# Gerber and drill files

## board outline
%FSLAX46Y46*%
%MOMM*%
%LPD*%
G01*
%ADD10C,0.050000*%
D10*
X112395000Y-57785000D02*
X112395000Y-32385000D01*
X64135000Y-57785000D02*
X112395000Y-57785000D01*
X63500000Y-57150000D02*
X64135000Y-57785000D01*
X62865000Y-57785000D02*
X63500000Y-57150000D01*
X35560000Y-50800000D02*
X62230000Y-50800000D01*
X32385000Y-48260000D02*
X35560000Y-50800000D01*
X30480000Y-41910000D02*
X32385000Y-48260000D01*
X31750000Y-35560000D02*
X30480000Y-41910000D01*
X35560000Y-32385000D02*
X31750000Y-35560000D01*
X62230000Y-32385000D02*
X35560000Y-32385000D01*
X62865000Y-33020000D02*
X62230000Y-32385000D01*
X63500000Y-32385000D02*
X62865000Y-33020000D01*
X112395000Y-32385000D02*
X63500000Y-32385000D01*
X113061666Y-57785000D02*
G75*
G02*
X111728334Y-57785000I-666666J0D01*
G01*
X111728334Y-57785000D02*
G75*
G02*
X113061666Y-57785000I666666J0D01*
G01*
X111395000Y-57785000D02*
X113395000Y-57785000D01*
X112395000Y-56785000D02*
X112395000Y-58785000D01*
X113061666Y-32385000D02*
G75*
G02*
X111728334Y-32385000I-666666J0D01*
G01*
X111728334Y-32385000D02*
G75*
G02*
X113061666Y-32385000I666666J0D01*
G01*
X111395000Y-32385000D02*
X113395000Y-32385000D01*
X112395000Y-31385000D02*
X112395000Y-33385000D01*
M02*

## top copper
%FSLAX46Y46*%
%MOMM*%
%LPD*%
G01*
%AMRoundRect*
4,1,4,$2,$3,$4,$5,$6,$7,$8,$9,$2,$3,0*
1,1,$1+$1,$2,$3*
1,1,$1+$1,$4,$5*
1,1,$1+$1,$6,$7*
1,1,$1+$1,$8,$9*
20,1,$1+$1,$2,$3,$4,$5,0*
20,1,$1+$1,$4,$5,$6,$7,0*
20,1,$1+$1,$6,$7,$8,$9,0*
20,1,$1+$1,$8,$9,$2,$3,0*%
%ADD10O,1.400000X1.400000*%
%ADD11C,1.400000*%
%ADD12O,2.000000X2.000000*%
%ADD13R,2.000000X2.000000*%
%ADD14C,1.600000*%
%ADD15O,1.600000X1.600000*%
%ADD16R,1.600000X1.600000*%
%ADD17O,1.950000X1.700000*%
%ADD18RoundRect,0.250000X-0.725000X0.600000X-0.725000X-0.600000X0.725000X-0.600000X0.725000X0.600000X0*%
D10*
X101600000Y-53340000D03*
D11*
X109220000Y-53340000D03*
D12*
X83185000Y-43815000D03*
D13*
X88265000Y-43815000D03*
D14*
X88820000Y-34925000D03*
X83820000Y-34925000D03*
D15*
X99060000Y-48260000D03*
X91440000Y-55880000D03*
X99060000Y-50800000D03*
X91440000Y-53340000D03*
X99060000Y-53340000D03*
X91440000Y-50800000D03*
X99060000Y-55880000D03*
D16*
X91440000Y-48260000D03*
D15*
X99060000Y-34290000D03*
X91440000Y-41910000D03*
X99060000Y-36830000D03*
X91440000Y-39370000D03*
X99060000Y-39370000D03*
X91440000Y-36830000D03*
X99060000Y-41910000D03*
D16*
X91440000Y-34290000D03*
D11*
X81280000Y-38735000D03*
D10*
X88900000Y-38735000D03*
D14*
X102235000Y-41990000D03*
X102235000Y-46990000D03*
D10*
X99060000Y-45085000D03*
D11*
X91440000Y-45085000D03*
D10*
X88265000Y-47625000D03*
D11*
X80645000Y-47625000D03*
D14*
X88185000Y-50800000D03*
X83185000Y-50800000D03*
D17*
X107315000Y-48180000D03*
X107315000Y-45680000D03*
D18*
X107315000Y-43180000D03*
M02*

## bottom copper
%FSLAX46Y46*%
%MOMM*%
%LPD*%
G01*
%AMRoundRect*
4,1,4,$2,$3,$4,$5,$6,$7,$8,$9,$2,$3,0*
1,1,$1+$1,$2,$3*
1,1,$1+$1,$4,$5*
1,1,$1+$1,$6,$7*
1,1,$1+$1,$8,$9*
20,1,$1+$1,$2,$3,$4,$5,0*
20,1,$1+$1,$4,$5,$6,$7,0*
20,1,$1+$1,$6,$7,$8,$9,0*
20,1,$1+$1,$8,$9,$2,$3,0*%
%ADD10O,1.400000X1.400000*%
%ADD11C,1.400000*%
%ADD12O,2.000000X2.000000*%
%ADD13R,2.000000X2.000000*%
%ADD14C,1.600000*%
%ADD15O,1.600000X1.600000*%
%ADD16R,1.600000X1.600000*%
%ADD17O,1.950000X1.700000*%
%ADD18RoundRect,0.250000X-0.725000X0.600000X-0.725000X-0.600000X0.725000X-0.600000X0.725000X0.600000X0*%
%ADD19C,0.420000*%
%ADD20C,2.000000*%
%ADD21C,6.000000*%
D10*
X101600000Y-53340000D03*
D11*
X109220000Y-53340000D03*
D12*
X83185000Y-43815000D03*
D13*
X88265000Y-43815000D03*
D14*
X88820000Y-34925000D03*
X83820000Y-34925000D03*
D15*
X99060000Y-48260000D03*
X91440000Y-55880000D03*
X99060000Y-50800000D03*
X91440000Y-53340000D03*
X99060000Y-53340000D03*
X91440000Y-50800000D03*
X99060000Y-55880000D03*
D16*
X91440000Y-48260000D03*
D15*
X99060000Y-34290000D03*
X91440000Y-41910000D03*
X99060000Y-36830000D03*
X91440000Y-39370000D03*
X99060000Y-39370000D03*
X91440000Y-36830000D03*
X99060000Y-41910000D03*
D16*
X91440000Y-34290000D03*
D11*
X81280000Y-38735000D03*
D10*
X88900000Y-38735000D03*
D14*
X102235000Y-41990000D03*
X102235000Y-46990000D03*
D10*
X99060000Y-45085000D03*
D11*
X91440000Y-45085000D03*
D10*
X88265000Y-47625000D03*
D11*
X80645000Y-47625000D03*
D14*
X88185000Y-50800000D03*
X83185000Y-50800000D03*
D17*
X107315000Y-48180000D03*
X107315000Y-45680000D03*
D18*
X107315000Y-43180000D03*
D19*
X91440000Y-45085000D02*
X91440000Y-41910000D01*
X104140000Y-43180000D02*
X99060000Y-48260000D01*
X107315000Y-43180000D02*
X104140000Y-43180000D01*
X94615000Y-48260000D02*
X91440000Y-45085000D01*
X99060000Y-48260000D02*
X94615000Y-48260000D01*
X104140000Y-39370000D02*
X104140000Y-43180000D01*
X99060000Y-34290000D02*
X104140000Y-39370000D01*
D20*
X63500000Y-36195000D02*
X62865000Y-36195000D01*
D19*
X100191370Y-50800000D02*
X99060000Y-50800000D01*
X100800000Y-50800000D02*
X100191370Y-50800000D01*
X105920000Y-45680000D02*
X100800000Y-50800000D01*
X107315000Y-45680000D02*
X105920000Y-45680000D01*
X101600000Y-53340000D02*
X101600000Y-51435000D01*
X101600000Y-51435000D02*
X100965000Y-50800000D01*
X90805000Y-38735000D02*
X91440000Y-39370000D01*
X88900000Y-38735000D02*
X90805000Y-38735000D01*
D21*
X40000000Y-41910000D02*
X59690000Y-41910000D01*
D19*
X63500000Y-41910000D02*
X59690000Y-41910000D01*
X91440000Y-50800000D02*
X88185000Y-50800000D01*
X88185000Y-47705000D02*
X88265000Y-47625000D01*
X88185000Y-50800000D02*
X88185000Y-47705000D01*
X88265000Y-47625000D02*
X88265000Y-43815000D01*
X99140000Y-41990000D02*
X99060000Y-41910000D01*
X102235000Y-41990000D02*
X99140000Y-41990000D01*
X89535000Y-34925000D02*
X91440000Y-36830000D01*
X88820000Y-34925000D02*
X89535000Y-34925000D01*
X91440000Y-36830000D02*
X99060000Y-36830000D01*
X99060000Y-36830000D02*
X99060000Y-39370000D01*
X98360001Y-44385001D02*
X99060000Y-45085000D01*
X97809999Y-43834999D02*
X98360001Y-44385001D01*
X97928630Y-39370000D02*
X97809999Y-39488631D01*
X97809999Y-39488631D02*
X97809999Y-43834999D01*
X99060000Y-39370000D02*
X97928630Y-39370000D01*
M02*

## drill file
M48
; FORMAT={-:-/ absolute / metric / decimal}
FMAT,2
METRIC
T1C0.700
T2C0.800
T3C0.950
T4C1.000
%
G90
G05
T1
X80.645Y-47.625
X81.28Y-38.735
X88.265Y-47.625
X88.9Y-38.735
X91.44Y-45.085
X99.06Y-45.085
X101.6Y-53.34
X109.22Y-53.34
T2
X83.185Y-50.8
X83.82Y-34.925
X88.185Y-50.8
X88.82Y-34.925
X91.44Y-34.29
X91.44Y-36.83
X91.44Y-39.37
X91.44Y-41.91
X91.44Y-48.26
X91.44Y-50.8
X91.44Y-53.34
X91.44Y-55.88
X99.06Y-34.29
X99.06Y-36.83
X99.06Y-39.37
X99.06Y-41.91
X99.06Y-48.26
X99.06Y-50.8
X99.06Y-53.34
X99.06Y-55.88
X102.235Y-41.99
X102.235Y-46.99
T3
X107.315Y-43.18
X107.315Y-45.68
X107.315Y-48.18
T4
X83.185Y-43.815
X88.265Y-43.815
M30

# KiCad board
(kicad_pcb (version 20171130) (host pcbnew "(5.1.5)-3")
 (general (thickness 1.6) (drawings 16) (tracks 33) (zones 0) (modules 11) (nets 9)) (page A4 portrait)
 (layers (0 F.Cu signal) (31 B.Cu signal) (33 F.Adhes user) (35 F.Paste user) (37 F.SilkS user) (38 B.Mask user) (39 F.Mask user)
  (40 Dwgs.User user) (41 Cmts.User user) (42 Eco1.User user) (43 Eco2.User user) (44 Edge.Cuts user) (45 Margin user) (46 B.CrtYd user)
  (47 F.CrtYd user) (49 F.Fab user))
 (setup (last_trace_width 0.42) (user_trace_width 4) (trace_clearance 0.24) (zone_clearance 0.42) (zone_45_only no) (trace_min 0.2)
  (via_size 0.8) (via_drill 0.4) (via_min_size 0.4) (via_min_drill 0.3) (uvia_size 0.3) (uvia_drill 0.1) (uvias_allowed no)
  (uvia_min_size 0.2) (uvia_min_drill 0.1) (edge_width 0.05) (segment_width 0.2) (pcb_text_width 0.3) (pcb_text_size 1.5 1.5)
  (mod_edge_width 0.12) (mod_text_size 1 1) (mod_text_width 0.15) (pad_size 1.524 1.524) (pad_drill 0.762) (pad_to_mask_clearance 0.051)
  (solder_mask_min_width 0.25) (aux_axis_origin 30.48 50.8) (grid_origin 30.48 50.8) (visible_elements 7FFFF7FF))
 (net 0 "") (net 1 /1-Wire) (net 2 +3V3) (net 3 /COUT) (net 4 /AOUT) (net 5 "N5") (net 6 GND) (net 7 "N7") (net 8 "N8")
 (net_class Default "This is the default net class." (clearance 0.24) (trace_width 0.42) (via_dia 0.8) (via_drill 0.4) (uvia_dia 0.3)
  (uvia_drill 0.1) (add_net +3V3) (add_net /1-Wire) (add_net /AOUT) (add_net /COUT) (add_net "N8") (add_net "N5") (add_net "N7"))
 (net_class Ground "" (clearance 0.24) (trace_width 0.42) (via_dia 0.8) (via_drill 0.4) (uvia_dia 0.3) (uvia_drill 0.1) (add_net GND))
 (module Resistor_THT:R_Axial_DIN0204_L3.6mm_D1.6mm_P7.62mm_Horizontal (layer F.Cu) (at 109.22 53.34 180)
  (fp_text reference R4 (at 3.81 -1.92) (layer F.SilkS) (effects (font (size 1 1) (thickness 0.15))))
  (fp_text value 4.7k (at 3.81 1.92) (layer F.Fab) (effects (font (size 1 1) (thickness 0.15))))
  (pad 2 thru_hole oval (at 7.62 0 180) (size 1.4 1.4) (drill 0.7) (layers *.Cu *.Mask) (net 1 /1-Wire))
  (pad 1 thru_hole circle (at 0 0 180) (size 1.4 1.4) (drill 0.7) (layers *.Cu *.Mask) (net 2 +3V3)))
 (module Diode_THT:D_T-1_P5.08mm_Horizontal (layer F.Cu) (at 88.265 43.815 180)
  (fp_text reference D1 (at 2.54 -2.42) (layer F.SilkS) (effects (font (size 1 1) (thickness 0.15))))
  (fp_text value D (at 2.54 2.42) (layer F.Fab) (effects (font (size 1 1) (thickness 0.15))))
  (pad 2 thru_hole oval (at 5.08 0 180) (size 2 2) (drill 1) (layers *.Cu *.Mask) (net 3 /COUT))
  (pad 1 thru_hole rect (at 0 0 180) (size 2 2) (drill 1) (layers *.Cu *.Mask) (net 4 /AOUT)))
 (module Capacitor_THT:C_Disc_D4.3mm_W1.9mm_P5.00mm (layer F.Cu) (at 83.82 34.925)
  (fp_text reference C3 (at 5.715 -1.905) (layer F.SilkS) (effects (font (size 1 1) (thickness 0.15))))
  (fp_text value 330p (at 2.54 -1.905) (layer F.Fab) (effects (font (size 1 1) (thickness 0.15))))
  (pad 2 thru_hole circle (at 5 0) (size 1.6 1.6) (drill 0.8) (layers *.Cu *.Mask) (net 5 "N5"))
  (pad 1 thru_hole circle (at 0 0) (size 1.6 1.6) (drill 0.8) (layers *.Cu *.Mask) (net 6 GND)))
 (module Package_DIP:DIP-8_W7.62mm (layer F.Cu) (at 91.44 48.26)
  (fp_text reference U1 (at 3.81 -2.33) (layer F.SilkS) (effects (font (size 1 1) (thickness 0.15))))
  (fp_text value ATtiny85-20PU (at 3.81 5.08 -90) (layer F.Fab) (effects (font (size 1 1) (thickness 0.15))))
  (pad 8 thru_hole oval (at 7.62 0) (size 1.6 1.6) (drill 0.8) (layers *.Cu *.Mask) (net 2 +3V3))
  (pad 4 thru_hole oval (at 0 7.62) (size 1.6 1.6) (drill 0.8) (layers *.Cu *.Mask) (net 6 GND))
  (pad 7 thru_hole oval (at 7.62 2.54) (size 1.6 1.6) (drill 0.8) (layers *.Cu *.Mask) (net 1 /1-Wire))
  (pad 3 thru_hole oval (at 0 5.08) (size 1.6 1.6) (drill 0.8) (layers *.Cu *.Mask) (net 6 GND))
  (pad 6 thru_hole oval (at 7.62 5.08) (size 1.6 1.6) (drill 0.8) (layers *.Cu *.Mask))
  (pad 2 thru_hole oval (at 0 2.54) (size 1.6 1.6) (drill 0.8) (layers *.Cu *.Mask) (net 4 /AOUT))
  (pad 5 thru_hole oval (at 7.62 7.62) (size 1.6 1.6) (drill 0.8) (layers *.Cu *.Mask))
  (pad 1 thru_hole rect (at 0 0) (size 1.6 1.6) (drill 0.8) (layers *.Cu *.Mask)))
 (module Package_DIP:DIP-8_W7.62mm (layer F.Cu) (at 91.44 34.29)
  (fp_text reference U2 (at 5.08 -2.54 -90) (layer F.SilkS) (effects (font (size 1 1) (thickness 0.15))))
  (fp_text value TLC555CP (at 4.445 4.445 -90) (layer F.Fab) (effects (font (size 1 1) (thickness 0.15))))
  (pad 8 thru_hole oval (at 7.62 0) (size 1.6 1.6) (drill 0.8) (layers *.Cu *.Mask) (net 2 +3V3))
  (pad 4 thru_hole oval (at 0 7.62) (size 1.6 1.6) (drill 0.8) (layers *.Cu *.Mask) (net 2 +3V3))
  (pad 7 thru_hole oval (at 7.62 2.54) (size 1.6 1.6) (drill 0.8) (layers *.Cu *.Mask) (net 5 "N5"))
  (pad 3 thru_hole oval (at 0 5.08) (size 1.6 1.6) (drill 0.8) (layers *.Cu *.Mask) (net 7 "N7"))
  (pad 6 thru_hole oval (at 7.62 5.08) (size 1.6 1.6) (drill 0.8) (layers *.Cu *.Mask) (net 5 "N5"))
  (pad 2 thru_hole oval (at 0 2.54) (size 1.6 1.6) (drill 0.8) (layers *.Cu *.Mask) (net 5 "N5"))
  (pad 5 thru_hole oval (at 7.62 7.62) (size 1.6 1.6) (drill 0.8) (layers *.Cu *.Mask) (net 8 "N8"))
  (pad 1 thru_hole rect (at 0 0) (size 1.6 1.6) (drill 0.8) (layers *.Cu *.Mask) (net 6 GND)))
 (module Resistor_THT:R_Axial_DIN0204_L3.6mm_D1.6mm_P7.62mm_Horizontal (layer F.Cu) (at 81.28 38.735)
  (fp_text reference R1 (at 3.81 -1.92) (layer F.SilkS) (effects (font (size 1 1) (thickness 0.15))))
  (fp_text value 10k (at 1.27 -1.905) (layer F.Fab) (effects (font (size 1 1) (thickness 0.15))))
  (pad 1 thru_hole circle (at 0 0) (size 1.4 1.4) (drill 0.7) (layers *.Cu *.Mask) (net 3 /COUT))
  (pad 2 thru_hole oval (at 7.62 0) (size 1.4 1.4) (drill 0.7) (layers *.Cu *.Mask) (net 7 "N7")))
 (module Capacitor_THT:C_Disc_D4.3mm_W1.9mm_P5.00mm (layer F.Cu) (at 102.235 46.99 90)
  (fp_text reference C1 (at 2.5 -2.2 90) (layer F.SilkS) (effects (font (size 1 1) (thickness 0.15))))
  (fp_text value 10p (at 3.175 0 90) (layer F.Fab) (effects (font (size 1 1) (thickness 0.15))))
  (pad 2 thru_hole circle (at 5 0 90) (size 1.6 1.6) (drill 0.8) (layers *.Cu *.Mask) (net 8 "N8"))
  (pad 1 thru_hole circle (at 0 0 90) (size 1.6 1.6) (drill 0.8) (layers *.Cu *.Mask) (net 6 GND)))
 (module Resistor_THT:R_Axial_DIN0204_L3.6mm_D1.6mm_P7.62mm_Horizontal (layer F.Cu) (at 91.44 45.085)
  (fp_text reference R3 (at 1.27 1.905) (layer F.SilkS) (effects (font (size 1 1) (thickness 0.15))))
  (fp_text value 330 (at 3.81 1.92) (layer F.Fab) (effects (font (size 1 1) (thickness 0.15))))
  (pad 2 thru_hole oval (at 7.62 0) (size 1.4 1.4) (drill 0.7) (layers *.Cu *.Mask) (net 5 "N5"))
  (pad 1 thru_hole circle (at 0 0) (size 1.4 1.4) (drill 0.7) (layers *.Cu *.Mask) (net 2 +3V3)))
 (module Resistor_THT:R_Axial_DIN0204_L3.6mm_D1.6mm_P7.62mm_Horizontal (layer F.Cu) (at 80.645 47.625)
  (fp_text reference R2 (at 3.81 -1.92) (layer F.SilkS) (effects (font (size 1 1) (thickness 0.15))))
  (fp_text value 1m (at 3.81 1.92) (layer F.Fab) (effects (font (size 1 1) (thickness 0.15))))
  (pad 2 thru_hole oval (at 7.62 0) (size 1.4 1.4) (drill 0.7) (layers *.Cu *.Mask) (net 4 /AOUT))
  (pad 1 thru_hole circle (at 0 0) (size 1.4 1.4) (drill 0.7) (layers *.Cu *.Mask) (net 6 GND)))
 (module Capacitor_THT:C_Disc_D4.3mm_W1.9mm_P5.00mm (layer F.Cu) (at 83.185 50.8)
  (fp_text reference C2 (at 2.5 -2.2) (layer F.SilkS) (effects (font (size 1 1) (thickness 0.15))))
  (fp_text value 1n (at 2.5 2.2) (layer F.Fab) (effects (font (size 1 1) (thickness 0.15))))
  (pad 2 thru_hole circle (at 5 0) (size 1.6 1.6) (drill 0.8) (layers *.Cu *.Mask) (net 4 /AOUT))
  (pad 1 thru_hole circle (at 0 0) (size 1.6 1.6) (drill 0.8) (layers *.Cu *.Mask) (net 6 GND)))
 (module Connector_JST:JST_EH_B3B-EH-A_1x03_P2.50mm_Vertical (layer F.Cu) (at 107.315 43.18 270)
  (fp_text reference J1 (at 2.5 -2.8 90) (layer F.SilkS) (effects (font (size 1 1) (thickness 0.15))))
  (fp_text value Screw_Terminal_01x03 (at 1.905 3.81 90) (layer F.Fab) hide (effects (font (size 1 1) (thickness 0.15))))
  (pad 3 thru_hole oval (at 5 0 270) (size 1.7 1.95) (drill 0.95) (layers *.Cu *.Mask) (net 6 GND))
  (pad 2 thru_hole oval (at 2.5 0 270) (size 1.7 1.95) (drill 0.95) (layers *.Cu *.Mask) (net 1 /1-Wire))
  (pad 1 thru_hole roundrect (at 0 0 270) (size 1.7 1.95) (drill 0.95) (layers *.Cu *.Mask) (roundrect_rratio 0.1470588235294118)
   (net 2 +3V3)))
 (gr_line (start 112.395 57.785) (end 112.395 32.385) (layer Edge.Cuts) (width 0.05))
 (gr_line (start 64.135 57.785) (end 112.395 57.785) (layer Edge.Cuts) (width 0.05))
 (gr_line (start 63.5 57.15) (end 64.135 57.785) (layer Edge.Cuts) (width 0.05))
 (gr_line (start 62.865 57.785) (end 63.5 57.15) (layer Edge.Cuts) (width 0.05))
 (gr_line (start 35.56 50.8) (end 62.23 50.8) (layer Edge.Cuts) (width 0.05))
 (gr_line (start 32.385 48.26) (end 35.56 50.8) (layer Edge.Cuts) (width 0.05))
 (gr_line (start 30.48 41.91) (end 32.385 48.26) (layer Edge.Cuts) (width 0.05))
 (gr_line (start 31.75 35.56) (end 30.48 41.91) (layer Edge.Cuts) (width 0.05))
 (gr_line (start 35.56 32.385) (end 31.75 35.56) (layer Edge.Cuts) (width 0.05))
 (gr_line (start 62.23 32.385) (end 35.56 32.385) (layer Edge.Cuts) (width 0.05))
 (gr_line (start 62.865 33.02) (end 62.23 32.385) (layer Edge.Cuts) (width 0.05))
 (gr_line (start 63.5 32.385) (end 62.865 33.02) (layer Edge.Cuts) (width 0.05))
 (gr_line (start 112.395 32.385) (end 63.5 32.385) (layer Edge.Cuts) (width 0.05))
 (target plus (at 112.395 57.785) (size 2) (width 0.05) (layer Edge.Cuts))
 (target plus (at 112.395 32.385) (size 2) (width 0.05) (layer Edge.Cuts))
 (segment (start 91.44 45.085) (end 91.44 41.91) (width 0.42) (layer B.Cu) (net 2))
 (segment (start 104.14 43.18) (end 99.06 48.26) (width 0.42) (layer B.Cu) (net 2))
 (segment (start 107.315 43.18) (end 104.14 43.18) (width 0.42) (layer B.Cu) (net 2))
 (segment (start 94.615 48.26) (end 91.44 45.085) (width 0.42) (layer B.Cu) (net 2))
 (segment (start 99.06 48.26) (end 94.615 48.26) (width 0.42) (layer B.Cu) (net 2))
 (segment (start 104.14 39.37) (end 104.14 43.18) (width 0.42) (layer B.Cu) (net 2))
 (segment (start 99.06 34.29) (end 104.14 39.37) (width 0.42) (layer B.Cu) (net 2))
 (segment (start 63.5 36.195) (end 62.865 36.195) (width 2) (layer B.Cu) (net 6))
 (segment (start 100.19137 50.8) (end 99.06 50.8) (width 0.42) (layer B.Cu) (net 1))
 (segment (start 100.8 50.8) (end 100.19137 50.8) (width 0.42) (layer B.Cu) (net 1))
 (segment (start 105.92 45.68) (end 100.8 50.8) (width 0.42) (layer B.Cu) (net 1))
 (segment (start 107.315 45.68) (end 105.92 45.68) (width 0.42) (layer B.Cu) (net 1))
 (segment (start 101.6 53.34) (end 101.6 51.435) (width 0.42) (layer B.Cu) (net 1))
 (segment (start 101.6 51.435) (end 100.965 50.8) (width 0.42) (layer B.Cu) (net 1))
 (segment (start 90.805 38.735) (end 91.44 39.37) (width 0.42) (layer B.Cu) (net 7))
 (segment (start 88.9 38.735) (end 90.805 38.735) (width 0.42) (layer B.Cu) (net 7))
 (segment (start 40 41.91) (end 59.69 41.91) (width 6) (layer B.Cu) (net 4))
 (segment (start 63.5 41.91) (end 59.69 41.91) (width 0.42) (layer B.Cu) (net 4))
 (segment (start 91.44 50.8) (end 88.185 50.8) (width 0.42) (layer B.Cu) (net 4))
 (segment (start 88.185 47.705) (end 88.265 47.625) (width 0.42) (layer B.Cu) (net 4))
 (segment (start 88.185 50.8) (end 88.185 47.705) (width 0.42) (layer B.Cu) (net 4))
 (segment (start 88.265 47.625) (end 88.265 43.815) (width 0.42) (layer B.Cu) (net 4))
 (segment (start 99.14 41.99) (end 99.06 41.91) (width 0.42) (layer B.Cu) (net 8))
 (segment (start 102.235 41.99) (end 99.14 41.99) (width 0.42) (layer B.Cu) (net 8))
 (segment (start 89.535 34.925) (end 91.44 36.83) (width 0.42) (layer B.Cu) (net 5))
 (segment (start 88.82 34.925) (end 89.535 34.925) (width 0.42) (layer B.Cu) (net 5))
 (segment (start 91.44 36.83) (end 99.06 36.83) (width 0.42) (layer B.Cu) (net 5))
 (segment (start 99.06 36.83) (end 99.06 39.37) (width 0.42) (layer B.Cu) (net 5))
 (segment (start 98.360001 44.385001) (end 99.06 45.085) (width 0.42) (layer B.Cu) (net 5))
 (segment (start 97.809999 43.834999) (end 98.360001 44.385001) (width 0.42) (layer B.Cu) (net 5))
 (segment (start 97.92863 39.37) (end 97.809999 39.488631) (width 0.42) (layer B.Cu) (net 5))
 (segment (start 97.809999 39.488631) (end 97.809999 43.834999) (width 0.42) (layer B.Cu) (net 5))
 (segment (start 99.06 39.37) (end 97.92863 39.37) (width 0.42) (layer B.Cu) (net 5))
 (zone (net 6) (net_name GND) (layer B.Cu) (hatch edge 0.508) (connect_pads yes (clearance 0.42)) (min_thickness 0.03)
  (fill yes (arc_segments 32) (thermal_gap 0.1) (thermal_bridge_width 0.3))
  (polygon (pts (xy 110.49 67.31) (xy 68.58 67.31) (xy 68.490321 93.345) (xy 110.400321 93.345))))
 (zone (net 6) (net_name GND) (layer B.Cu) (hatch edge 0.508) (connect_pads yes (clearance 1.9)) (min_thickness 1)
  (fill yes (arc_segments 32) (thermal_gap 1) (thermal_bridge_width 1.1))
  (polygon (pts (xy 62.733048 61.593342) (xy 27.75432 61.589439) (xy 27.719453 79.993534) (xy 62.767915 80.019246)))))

